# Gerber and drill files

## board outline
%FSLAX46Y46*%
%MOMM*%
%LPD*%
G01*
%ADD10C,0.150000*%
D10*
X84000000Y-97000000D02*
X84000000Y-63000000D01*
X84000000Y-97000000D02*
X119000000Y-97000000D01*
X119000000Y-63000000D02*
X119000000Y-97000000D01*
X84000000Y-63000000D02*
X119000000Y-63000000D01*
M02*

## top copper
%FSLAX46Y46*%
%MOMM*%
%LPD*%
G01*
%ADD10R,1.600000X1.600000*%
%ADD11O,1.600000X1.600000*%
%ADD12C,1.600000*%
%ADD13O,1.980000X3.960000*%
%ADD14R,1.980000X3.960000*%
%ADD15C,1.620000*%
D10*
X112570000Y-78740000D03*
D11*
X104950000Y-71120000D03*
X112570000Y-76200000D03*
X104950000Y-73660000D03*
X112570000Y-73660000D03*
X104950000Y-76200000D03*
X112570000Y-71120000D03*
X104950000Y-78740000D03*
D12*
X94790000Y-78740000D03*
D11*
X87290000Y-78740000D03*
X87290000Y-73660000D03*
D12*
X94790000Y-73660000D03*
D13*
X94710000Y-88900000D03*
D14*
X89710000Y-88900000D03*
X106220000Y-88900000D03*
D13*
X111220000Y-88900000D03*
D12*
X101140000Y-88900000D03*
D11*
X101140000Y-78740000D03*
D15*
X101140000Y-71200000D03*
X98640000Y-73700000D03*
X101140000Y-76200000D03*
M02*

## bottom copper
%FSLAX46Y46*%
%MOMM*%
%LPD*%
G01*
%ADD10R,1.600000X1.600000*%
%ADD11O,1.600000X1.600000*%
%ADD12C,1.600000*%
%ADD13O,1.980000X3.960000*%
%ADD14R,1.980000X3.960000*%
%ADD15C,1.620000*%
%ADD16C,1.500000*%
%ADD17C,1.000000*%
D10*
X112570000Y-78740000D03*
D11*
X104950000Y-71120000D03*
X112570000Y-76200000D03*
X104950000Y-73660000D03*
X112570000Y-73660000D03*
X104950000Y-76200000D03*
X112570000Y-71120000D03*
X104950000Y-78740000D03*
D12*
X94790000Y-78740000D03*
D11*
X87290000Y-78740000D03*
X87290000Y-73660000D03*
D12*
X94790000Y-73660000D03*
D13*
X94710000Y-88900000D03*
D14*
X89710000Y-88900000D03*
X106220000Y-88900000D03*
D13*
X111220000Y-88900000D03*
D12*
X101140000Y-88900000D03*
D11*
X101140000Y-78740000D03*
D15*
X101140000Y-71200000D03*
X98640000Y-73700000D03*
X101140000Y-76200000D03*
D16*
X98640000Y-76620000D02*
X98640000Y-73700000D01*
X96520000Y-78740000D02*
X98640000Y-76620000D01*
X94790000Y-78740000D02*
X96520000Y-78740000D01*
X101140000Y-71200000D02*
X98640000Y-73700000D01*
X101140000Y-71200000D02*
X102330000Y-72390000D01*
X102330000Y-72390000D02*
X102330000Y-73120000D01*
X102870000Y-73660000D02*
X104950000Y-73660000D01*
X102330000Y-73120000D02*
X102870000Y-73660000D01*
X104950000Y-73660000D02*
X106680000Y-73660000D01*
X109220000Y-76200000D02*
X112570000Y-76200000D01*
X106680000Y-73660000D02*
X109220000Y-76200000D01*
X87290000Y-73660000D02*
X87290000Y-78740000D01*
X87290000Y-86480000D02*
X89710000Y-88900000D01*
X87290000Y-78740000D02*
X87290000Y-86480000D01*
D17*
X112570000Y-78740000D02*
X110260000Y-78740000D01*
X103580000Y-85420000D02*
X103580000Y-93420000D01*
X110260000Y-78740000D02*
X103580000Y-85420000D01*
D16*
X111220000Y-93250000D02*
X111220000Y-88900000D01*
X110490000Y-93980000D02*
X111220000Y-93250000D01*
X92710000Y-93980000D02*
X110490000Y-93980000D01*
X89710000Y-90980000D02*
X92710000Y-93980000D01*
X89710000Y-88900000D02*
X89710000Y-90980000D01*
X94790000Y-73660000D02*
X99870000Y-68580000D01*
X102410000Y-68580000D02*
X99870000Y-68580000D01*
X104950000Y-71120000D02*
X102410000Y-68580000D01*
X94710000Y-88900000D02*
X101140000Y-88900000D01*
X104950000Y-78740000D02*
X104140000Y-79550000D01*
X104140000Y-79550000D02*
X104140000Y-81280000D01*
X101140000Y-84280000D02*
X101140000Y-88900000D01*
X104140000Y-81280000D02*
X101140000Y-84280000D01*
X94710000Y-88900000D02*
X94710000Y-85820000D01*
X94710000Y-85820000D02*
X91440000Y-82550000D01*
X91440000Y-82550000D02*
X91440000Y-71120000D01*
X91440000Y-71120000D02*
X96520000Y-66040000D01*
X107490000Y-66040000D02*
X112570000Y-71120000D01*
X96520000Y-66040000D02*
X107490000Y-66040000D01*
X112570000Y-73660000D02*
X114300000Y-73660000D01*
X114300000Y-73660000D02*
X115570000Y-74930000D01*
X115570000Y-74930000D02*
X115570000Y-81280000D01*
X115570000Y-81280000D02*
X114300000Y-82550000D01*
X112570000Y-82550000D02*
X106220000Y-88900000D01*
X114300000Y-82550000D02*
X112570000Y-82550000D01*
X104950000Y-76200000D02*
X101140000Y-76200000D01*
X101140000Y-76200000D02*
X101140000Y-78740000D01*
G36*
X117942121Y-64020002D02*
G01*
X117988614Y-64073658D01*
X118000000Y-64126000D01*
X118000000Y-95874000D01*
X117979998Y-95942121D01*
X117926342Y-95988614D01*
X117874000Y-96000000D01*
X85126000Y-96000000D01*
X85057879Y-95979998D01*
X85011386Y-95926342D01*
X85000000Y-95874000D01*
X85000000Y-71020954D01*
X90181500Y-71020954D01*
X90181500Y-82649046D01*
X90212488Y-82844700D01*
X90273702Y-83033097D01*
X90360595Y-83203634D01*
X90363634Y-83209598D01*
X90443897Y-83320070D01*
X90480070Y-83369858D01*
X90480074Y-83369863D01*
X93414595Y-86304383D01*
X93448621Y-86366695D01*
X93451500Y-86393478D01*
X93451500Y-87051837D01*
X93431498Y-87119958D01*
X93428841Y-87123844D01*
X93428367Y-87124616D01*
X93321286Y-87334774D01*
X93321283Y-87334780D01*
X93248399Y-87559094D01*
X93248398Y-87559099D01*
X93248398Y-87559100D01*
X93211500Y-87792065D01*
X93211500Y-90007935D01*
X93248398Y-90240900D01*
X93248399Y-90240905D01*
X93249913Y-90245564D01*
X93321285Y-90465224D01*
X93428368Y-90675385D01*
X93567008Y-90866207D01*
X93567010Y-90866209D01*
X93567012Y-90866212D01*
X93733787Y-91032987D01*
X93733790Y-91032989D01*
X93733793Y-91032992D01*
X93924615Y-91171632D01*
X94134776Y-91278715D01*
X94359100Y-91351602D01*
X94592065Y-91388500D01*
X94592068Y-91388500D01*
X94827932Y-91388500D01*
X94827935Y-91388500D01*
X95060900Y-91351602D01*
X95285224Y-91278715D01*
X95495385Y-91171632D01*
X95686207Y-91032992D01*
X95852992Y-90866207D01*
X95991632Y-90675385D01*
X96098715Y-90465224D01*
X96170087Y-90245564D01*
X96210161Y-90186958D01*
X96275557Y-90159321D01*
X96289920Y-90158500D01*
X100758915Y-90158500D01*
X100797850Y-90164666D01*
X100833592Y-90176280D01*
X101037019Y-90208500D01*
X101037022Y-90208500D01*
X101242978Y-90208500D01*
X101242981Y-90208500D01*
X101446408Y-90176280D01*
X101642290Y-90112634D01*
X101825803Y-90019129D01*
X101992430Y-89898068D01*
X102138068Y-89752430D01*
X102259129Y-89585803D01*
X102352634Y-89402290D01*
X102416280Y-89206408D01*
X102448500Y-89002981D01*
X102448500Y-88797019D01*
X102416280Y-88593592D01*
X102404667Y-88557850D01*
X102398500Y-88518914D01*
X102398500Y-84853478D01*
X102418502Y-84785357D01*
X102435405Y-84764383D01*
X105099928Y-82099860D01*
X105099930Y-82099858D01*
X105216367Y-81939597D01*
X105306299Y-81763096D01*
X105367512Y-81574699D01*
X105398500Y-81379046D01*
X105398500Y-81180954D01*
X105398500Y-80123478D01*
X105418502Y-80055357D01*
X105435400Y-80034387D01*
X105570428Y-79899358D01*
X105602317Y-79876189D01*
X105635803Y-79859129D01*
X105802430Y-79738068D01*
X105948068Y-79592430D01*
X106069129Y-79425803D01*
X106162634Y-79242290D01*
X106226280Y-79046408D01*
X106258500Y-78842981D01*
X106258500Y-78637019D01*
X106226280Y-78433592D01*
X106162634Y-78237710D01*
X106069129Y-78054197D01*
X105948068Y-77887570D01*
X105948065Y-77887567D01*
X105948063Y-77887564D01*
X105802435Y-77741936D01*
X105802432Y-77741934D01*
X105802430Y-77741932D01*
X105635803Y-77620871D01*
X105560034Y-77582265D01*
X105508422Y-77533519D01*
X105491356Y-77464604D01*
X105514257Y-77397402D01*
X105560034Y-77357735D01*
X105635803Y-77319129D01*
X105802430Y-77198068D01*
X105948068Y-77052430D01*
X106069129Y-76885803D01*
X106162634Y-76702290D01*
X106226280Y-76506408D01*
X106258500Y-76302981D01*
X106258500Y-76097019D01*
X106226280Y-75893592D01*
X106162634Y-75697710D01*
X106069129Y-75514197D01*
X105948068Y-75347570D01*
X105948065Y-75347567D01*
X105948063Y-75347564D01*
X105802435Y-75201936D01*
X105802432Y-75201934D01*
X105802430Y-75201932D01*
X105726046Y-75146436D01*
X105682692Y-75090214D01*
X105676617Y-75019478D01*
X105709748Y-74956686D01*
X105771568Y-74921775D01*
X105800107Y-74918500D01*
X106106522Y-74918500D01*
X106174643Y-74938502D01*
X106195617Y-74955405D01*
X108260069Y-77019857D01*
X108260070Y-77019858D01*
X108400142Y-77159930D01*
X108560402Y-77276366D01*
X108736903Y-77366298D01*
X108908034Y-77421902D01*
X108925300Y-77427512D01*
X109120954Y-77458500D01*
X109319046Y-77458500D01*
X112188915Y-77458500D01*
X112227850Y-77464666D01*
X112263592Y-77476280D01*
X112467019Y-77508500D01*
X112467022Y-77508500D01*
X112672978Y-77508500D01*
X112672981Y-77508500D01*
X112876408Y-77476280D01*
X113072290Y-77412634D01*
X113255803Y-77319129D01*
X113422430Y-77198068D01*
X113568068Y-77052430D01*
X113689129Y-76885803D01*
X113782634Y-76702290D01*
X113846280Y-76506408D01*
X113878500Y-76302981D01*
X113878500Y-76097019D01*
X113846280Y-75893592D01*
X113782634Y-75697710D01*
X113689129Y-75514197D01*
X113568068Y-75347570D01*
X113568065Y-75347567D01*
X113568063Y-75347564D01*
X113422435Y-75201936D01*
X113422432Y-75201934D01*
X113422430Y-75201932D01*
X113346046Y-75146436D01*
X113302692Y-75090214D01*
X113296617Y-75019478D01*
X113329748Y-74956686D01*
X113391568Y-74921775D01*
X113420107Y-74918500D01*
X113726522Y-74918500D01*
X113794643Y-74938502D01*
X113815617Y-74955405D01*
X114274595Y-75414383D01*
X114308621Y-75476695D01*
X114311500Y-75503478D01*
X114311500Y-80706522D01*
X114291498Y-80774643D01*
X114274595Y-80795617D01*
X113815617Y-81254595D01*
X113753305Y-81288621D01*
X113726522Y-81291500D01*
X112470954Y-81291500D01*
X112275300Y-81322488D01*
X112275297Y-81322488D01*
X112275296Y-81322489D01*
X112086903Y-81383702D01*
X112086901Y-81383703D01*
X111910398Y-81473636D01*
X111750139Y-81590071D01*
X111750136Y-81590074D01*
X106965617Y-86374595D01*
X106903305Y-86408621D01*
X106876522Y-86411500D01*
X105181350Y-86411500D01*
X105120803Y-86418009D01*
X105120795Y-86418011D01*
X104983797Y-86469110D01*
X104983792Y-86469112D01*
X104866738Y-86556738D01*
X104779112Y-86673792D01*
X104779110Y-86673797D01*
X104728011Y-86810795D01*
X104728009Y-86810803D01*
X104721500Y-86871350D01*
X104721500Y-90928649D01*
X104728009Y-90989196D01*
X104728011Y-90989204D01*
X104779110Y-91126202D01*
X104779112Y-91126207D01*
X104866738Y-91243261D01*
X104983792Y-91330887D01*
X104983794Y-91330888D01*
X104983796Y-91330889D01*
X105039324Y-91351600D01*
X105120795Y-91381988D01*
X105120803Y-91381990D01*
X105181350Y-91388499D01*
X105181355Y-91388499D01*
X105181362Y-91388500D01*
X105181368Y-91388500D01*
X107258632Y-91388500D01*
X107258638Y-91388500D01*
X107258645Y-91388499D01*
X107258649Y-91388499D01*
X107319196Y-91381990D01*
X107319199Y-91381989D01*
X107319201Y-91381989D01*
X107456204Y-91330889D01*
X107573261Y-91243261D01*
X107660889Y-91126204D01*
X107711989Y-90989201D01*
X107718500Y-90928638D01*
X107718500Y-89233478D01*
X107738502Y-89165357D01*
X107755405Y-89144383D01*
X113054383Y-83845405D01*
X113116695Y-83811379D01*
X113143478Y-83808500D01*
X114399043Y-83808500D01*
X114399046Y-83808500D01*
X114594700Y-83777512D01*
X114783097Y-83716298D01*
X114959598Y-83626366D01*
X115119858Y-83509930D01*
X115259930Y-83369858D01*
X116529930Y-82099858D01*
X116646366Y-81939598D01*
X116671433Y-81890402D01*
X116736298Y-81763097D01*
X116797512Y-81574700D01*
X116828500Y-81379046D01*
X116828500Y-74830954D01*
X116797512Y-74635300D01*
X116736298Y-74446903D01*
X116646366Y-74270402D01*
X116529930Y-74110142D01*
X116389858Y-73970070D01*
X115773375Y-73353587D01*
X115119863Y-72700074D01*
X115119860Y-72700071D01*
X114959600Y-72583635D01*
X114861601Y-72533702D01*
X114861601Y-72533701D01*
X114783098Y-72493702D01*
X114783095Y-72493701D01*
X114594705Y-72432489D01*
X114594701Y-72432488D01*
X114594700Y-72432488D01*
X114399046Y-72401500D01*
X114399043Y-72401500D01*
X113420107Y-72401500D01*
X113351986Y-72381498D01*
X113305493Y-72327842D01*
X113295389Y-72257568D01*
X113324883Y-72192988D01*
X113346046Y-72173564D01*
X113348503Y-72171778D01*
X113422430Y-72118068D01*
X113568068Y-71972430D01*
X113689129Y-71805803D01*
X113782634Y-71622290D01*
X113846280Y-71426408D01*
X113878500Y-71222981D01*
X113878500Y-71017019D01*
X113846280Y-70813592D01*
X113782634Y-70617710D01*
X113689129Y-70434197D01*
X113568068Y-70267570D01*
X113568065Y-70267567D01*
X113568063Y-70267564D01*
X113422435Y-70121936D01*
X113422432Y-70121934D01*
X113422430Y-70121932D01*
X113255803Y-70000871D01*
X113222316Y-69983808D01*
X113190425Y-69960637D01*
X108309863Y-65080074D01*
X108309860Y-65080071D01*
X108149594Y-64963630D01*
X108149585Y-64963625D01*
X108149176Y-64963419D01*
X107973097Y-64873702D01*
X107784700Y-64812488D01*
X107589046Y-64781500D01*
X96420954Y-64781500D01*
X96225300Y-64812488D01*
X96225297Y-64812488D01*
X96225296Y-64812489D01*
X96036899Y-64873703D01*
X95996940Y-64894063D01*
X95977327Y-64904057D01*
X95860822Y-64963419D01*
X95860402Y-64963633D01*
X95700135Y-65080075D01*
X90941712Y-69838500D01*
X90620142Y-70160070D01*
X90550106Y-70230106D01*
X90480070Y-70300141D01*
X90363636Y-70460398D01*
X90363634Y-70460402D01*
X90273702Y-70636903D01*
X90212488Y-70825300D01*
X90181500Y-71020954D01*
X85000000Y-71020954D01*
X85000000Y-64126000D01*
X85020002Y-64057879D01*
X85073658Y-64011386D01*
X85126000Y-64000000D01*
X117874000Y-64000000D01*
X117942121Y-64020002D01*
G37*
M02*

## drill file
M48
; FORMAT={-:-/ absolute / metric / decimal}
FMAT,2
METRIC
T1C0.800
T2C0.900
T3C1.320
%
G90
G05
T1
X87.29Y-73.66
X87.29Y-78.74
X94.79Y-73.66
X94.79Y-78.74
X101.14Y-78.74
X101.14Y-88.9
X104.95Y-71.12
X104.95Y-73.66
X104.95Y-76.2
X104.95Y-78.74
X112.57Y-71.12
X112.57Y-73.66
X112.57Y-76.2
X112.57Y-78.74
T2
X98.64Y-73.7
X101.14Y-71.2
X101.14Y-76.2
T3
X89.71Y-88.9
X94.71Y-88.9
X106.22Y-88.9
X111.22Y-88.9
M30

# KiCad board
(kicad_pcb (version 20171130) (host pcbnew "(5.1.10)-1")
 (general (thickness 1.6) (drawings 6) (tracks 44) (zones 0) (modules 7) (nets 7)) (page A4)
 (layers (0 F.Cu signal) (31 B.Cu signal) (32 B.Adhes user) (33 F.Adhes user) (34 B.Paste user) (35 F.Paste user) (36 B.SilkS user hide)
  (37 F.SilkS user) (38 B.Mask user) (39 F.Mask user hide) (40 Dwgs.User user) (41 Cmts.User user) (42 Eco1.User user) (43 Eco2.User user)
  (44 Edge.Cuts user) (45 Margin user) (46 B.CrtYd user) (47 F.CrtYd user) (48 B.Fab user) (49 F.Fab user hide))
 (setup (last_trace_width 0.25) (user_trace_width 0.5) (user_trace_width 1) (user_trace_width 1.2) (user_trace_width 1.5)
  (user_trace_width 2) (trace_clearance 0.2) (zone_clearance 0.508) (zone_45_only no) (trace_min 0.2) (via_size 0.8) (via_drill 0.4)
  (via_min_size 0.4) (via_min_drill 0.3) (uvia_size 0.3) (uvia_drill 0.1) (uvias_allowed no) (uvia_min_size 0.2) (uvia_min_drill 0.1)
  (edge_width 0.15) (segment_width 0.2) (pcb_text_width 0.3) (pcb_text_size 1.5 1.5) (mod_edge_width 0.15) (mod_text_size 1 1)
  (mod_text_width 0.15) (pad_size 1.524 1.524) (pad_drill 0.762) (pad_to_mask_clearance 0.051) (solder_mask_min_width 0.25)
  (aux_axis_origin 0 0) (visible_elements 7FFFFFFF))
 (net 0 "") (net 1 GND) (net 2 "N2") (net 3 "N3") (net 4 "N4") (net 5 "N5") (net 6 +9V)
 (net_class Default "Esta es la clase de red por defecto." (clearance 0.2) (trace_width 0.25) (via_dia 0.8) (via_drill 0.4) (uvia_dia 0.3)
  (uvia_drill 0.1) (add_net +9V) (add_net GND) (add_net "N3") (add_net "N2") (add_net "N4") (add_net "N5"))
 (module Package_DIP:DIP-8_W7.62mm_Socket (layer F.Cu) (at 112.57 78.74 180)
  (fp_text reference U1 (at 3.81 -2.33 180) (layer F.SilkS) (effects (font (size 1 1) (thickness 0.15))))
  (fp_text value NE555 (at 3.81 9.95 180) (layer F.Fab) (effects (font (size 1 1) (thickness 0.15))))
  (pad 1 thru_hole rect (at 0 0 180) (size 1.6 1.6) (drill 0.8) (layers *.Cu *.Mask) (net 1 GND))
  (pad 5 thru_hole oval (at 7.62 7.62 180) (size 1.6 1.6) (drill 0.8) (layers *.Cu *.Mask) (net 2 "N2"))
  (pad 2 thru_hole oval (at 0 2.54 180) (size 1.6 1.6) (drill 0.8) (layers *.Cu *.Mask) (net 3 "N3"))
  (pad 6 thru_hole oval (at 7.62 5.08 180) (size 1.6 1.6) (drill 0.8) (layers *.Cu *.Mask) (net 3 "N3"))
  (pad 3 thru_hole oval (at 0 5.08 180) (size 1.6 1.6) (drill 0.8) (layers *.Cu *.Mask) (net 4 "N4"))
  (pad 7 thru_hole oval (at 7.62 2.54 180) (size 1.6 1.6) (drill 0.8) (layers *.Cu *.Mask) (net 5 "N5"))
  (pad 4 thru_hole oval (at 0 7.62 180) (size 1.6 1.6) (drill 0.8) (layers *.Cu *.Mask) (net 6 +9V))
  (pad 8 thru_hole oval (at 7.62 0 180) (size 1.6 1.6) (drill 0.8) (layers *.Cu *.Mask) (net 6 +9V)))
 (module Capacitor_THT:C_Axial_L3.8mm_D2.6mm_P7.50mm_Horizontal (layer F.Cu) (at 94.79 78.74 180)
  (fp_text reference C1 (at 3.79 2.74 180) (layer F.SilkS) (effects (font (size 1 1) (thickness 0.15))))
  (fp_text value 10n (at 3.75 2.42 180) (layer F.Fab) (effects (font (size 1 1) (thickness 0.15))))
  (pad 1 thru_hole circle (at 0 0 180) (size 1.6 1.6) (drill 0.8) (layers *.Cu *.Mask) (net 3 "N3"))
  (pad 2 thru_hole oval (at 7.5 0 180) (size 1.6 1.6) (drill 0.8) (layers *.Cu *.Mask) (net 1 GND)))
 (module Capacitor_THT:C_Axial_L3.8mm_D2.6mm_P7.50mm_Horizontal (layer F.Cu) (at 94.79 73.66 180)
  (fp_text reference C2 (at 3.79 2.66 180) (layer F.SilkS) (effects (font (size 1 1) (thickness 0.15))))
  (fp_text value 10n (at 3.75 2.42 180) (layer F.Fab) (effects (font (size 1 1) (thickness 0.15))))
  (pad 2 thru_hole oval (at 7.5 0 180) (size 1.6 1.6) (drill 0.8) (layers *.Cu *.Mask) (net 1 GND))
  (pad 1 thru_hole circle (at 0 0 180) (size 1.6 1.6) (drill 0.8) (layers *.Cu *.Mask) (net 2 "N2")))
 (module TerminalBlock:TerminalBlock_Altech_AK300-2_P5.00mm (layer F.Cu) (at 89.71 88.9)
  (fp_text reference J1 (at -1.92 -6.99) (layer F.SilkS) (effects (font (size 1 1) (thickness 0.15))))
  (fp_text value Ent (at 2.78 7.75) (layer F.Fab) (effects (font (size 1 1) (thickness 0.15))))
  (pad 2 thru_hole oval (at 5 0) (size 1.98 3.96) (drill 1.32) (layers *.Cu *.Mask) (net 6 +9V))
  (pad 1 thru_hole rect (at 0 0) (size 1.98 3.96) (drill 1.32) (layers *.Cu *.Mask) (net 1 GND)))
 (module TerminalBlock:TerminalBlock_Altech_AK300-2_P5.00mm (layer F.Cu) (at 106.22 88.9)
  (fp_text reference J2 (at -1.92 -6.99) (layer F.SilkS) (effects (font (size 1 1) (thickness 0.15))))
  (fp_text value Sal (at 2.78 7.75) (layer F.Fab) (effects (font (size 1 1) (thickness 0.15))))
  (pad 1 thru_hole rect (at 0 0) (size 1.98 3.96) (drill 1.32) (layers *.Cu *.Mask) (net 4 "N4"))
  (pad 2 thru_hole oval (at 5 0) (size 1.98 3.96) (drill 1.32) (layers *.Cu *.Mask) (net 1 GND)))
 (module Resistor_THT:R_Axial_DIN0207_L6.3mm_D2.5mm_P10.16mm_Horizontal (layer F.Cu) (at 101.14 88.9 90)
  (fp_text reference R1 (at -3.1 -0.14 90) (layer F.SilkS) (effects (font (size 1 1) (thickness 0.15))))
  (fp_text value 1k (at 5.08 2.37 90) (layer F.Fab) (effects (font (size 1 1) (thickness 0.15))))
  (pad 1 thru_hole circle (at 0 0 90) (size 1.6 1.6) (drill 0.8) (layers *.Cu *.Mask) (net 6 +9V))
  (pad 2 thru_hole oval (at 10.16 0 90) (size 1.6 1.6) (drill 0.8) (layers *.Cu *.Mask) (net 5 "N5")))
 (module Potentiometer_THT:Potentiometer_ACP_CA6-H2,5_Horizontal (layer F.Cu) (at 101.14 76.2 180)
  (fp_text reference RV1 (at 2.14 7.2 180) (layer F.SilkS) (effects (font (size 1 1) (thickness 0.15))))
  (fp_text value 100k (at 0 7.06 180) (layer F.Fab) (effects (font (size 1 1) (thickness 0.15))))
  (pad 3 thru_hole circle (at 0 5 180) (size 1.62 1.62) (drill 0.9) (layers *.Cu *.Mask) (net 3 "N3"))
  (pad 2 thru_hole circle (at 2.5 2.5 180) (size 1.62 1.62) (drill 0.9) (layers *.Cu *.Mask) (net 3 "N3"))
  (pad 1 thru_hole circle (at 0 0 180) (size 1.62 1.62) (drill 0.9) (layers *.Cu *.Mask) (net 5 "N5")))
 (gr_line (start 84 97) (end 84 63) (layer Edge.Cuts) (width 0.15))
 (gr_line (start 84 97) (end 119 97) (layer Edge.Cuts) (width 0.15))
 (gr_line (start 119 63) (end 119 97) (layer Edge.Cuts) (width 0.15))
 (gr_line (start 84 63) (end 119 63) (layer Edge.Cuts) (width 0.15))
 (segment (start 98.64 76.62) (end 98.64 73.7) (width 1.5) (layer B.Cu) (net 3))
 (segment (start 96.52 78.74) (end 98.64 76.62) (width 1.5) (layer B.Cu) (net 3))
 (segment (start 94.79 78.74) (end 96.52 78.74) (width 1.5) (layer B.Cu) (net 3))
 (segment (start 101.14 71.2) (end 98.64 73.7) (width 1.5) (layer B.Cu) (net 3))
 (segment (start 101.14 71.2) (end 102.33 72.39) (width 1.5) (layer B.Cu) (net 3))
 (segment (start 102.33 72.39) (end 102.33 73.12) (width 1.5) (layer B.Cu) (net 3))
 (segment (start 102.87 73.66) (end 104.95 73.66) (width 1.5) (layer B.Cu) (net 3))
 (segment (start 102.33 73.12) (end 102.87 73.66) (width 1.5) (layer B.Cu) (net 3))
 (segment (start 104.95 73.66) (end 106.68 73.66) (width 1.5) (layer B.Cu) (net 3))
 (segment (start 109.22 76.2) (end 112.57 76.2) (width 1.5) (layer B.Cu) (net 3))
 (segment (start 106.68 73.66) (end 109.22 76.2) (width 1.5) (layer B.Cu) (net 3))
 (segment (start 87.29 73.66) (end 87.29 78.74) (width 1.5) (layer B.Cu) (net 1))
 (segment (start 87.29 86.48) (end 89.71 88.9) (width 1.5) (layer B.Cu) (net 1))
 (segment (start 87.29 78.74) (end 87.29 86.48) (width 1.5) (layer B.Cu) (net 1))
 (segment (start 112.57 78.74) (end 110.26 78.74) (width 1) (layer B.Cu) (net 1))
 (segment (start 103.58 85.42) (end 103.58 93.42) (width 1) (layer B.Cu) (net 1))
 (segment (start 110.26 78.74) (end 103.58 85.42) (width 1) (layer B.Cu) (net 1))
 (segment (start 111.22 93.25) (end 111.22 88.9) (width 1.5) (layer B.Cu) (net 1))
 (segment (start 110.49 93.98) (end 111.22 93.25) (width 1.5) (layer B.Cu) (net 1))
 (segment (start 92.71 93.98) (end 110.49 93.98) (width 1.5) (layer B.Cu) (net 1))
 (segment (start 89.71 90.98) (end 92.71 93.98) (width 1.5) (layer B.Cu) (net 1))
 (segment (start 89.71 88.9) (end 89.71 90.98) (width 1.5) (layer B.Cu) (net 1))
 (segment (start 94.79 73.66) (end 99.87 68.58) (width 1.5) (layer B.Cu) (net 2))
 (segment (start 102.41 68.58) (end 99.87 68.58) (width 1.5) (layer B.Cu) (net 2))
 (segment (start 104.95 71.12) (end 102.41 68.58) (width 1.5) (layer B.Cu) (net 2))
 (segment (start 94.71 88.9) (end 101.14 88.9) (width 1.5) (layer B.Cu) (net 6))
 (segment (start 104.95 78.74) (end 104.14 79.55) (width 1.5) (layer B.Cu) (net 6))
 (segment (start 104.14 79.55) (end 104.14 81.28) (width 1.5) (layer B.Cu) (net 6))
 (segment (start 101.14 84.28) (end 101.14 88.9) (width 1.5) (layer B.Cu) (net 6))
 (segment (start 104.14 81.28) (end 101.14 84.28) (width 1.5) (layer B.Cu) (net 6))
 (segment (start 94.71 88.9) (end 94.71 85.82) (width 1.5) (layer B.Cu) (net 6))
 (segment (start 94.71 85.82) (end 91.44 82.55) (width 1.5) (layer B.Cu) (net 6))
 (segment (start 91.44 82.55) (end 91.44 71.12) (width 1.5) (layer B.Cu) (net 6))
 (segment (start 91.44 71.12) (end 96.52 66.04) (width 1.5) (layer B.Cu) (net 6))
 (segment (start 107.49 66.04) (end 112.57 71.12) (width 1.5) (layer B.Cu) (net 6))
 (segment (start 96.52 66.04) (end 107.49 66.04) (width 1.5) (layer B.Cu) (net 6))
 (segment (start 112.57 73.66) (end 114.3 73.66) (width 1.5) (layer B.Cu) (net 4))
 (segment (start 114.3 73.66) (end 115.57 74.93) (width 1.5) (layer B.Cu) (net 4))
 (segment (start 115.57 74.93) (end 115.57 81.28) (width 1.5) (layer B.Cu) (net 4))
 (segment (start 115.57 81.28) (end 114.3 82.55) (width 1.5) (layer B.Cu) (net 4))
 (segment (start 112.57 82.55) (end 106.22 88.9) (width 1.5) (layer B.Cu) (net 4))
 (segment (start 114.3 82.55) (end 112.57 82.55) (width 1.5) (layer B.Cu) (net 4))
 (segment (start 104.95 76.2) (end 101.14 76.2) (width 1.5) (layer B.Cu) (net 5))
 (segment (start 101.14 76.2) (end 101.14 78.74) (width 1.5) (layer B.Cu) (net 5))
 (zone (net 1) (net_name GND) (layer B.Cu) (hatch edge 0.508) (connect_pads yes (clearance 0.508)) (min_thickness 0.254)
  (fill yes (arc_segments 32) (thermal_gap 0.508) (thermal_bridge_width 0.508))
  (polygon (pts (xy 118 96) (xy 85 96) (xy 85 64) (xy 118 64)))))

